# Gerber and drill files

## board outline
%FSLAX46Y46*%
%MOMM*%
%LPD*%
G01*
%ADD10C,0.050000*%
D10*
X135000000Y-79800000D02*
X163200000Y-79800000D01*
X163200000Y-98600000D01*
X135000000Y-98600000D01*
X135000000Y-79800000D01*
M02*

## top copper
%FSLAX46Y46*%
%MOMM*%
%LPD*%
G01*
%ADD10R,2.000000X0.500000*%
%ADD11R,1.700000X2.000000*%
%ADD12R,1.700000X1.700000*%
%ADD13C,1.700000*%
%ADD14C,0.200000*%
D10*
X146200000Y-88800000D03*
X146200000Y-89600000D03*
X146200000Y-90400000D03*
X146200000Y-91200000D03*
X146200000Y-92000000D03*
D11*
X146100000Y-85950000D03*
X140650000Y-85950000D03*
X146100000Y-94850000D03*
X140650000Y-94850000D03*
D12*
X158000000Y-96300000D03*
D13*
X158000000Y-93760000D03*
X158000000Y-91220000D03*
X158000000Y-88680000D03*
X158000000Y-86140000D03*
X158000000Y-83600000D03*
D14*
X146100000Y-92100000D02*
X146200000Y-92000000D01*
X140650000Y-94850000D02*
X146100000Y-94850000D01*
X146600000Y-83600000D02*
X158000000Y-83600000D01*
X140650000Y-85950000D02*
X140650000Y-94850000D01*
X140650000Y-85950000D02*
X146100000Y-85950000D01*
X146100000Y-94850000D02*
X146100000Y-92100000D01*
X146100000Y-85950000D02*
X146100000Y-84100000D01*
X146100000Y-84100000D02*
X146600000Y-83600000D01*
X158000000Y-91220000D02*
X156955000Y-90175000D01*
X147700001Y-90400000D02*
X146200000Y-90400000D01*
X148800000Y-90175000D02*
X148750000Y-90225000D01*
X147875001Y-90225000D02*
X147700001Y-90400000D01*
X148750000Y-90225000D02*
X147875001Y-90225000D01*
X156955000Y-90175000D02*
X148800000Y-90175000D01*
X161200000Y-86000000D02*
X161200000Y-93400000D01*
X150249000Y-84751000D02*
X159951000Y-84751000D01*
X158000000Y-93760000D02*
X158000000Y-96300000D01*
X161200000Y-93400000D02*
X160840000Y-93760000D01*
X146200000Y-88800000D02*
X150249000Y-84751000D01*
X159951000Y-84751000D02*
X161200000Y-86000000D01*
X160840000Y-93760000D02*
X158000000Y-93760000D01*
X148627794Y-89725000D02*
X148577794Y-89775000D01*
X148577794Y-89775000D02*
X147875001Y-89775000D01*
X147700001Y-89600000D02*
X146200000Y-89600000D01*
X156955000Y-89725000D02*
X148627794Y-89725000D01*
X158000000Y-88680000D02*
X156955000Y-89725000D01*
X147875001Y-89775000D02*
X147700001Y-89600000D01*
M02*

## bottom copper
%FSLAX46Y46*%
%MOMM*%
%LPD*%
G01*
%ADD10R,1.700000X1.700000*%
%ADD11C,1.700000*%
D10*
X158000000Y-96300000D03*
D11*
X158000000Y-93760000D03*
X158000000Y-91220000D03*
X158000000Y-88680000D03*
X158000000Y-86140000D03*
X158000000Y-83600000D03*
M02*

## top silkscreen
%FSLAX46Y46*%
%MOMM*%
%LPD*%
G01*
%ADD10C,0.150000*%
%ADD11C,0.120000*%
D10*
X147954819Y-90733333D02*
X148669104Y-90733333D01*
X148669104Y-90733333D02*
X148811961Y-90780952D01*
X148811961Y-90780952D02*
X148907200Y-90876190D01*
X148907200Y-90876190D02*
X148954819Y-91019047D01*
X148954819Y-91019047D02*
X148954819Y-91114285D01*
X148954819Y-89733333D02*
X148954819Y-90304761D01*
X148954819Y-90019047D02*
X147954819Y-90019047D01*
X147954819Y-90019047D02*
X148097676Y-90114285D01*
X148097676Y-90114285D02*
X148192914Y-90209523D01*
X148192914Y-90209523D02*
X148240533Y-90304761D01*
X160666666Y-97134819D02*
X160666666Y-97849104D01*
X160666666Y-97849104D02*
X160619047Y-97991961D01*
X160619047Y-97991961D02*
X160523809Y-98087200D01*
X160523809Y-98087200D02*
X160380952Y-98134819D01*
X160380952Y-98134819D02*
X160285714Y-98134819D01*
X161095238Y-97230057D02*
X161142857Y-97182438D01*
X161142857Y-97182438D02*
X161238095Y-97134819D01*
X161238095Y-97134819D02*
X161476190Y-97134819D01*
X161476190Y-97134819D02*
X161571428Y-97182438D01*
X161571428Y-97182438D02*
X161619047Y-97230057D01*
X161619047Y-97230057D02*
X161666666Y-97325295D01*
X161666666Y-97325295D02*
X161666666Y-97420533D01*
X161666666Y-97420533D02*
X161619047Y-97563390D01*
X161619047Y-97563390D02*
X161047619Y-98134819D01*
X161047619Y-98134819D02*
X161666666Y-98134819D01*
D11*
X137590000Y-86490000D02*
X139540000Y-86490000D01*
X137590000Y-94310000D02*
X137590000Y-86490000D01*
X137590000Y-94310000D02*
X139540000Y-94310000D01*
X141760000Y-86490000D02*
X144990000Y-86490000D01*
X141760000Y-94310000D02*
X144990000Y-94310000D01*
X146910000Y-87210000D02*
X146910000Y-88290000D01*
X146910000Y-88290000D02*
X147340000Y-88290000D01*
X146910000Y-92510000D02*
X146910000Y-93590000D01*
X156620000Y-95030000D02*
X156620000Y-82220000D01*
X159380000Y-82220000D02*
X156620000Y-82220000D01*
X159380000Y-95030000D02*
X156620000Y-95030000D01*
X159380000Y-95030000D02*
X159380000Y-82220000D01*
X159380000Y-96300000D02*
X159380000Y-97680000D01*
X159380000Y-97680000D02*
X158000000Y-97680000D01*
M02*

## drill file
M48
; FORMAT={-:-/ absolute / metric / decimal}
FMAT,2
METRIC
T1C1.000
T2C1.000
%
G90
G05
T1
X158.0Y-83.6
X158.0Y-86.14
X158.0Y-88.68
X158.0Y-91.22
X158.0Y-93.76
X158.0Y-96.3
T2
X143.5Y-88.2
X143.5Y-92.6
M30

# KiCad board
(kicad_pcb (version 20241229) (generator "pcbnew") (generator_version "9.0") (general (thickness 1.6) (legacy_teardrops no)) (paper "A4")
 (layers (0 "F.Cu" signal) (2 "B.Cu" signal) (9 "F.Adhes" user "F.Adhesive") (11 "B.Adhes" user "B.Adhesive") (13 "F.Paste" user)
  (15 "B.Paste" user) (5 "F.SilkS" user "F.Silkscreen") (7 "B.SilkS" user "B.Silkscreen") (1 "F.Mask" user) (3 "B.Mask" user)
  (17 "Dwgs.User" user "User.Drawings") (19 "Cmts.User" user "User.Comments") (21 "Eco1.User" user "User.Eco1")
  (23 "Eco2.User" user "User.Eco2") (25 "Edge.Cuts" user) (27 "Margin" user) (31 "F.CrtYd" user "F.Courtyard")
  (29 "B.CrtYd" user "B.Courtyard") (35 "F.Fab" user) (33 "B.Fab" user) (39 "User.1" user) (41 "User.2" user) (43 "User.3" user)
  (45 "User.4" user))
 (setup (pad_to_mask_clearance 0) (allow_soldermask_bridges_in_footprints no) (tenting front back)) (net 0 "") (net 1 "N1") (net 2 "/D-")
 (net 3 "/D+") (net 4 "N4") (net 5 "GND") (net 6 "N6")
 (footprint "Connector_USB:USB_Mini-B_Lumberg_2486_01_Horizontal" (layer "F.Cu") (at 143.5 90.4 -90)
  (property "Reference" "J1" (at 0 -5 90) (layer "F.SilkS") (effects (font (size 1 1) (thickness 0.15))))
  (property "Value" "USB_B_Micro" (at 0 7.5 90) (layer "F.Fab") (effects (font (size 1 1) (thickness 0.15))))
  (fp_line (start -3.91 5.91) (end -3.91 3.96) (stroke (width 0.12) (type solid)) (layer "F.SilkS"))
  (fp_line (start 3.91 5.91) (end -3.91 5.91) (stroke (width 0.12) (type solid)) (layer "F.SilkS"))
  (fp_line (start 3.91 5.91) (end 3.91 3.96) (stroke (width 0.12) (type solid)) (layer "F.SilkS"))
  (fp_line (start -3.91 1.74) (end -3.91 -1.49) (stroke (width 0.12) (type solid)) (layer "F.SilkS"))
  (fp_line (start 3.91 1.74) (end 3.91 -1.49) (stroke (width 0.12) (type solid)) (layer "F.SilkS"))
  (fp_line (start -3.19 -3.41) (end -2.11 -3.41) (stroke (width 0.12) (type solid)) (layer "F.SilkS"))
  (fp_line (start -2.11 -3.41) (end -2.11 -3.84) (stroke (width 0.12) (type solid)) (layer "F.SilkS"))
  (fp_line (start 2.11 -3.41) (end 3.19 -3.41) (stroke (width 0.12) (type solid)) (layer "F.SilkS"))
  (pad "" np_thru_hole circle (at -2.2 0 270) (size 1 1) (drill 1) (layers "*.Cu" "*.Mask"))
  (pad "" np_thru_hole circle (at 2.2 0 270) (size 1 1) (drill 1) (layers "*.Cu" "*.Mask"))
  (pad "1" smd rect (at -1.6 -2.7 270) (size 0.5 2) (layers "F.Cu" "F.Mask" "F.Paste") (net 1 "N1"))
  (pad "2" smd rect (at -0.8 -2.7 270) (size 0.5 2) (layers "F.Cu" "F.Mask" "F.Paste") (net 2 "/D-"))
  (pad "3" smd rect (at 0 -2.7 270) (size 0.5 2) (layers "F.Cu" "F.Mask" "F.Paste") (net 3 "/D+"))
  (pad "4" smd rect (at 0.8 -2.7 270) (size 0.5 2) (layers "F.Cu" "F.Mask" "F.Paste") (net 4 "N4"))
  (pad "5" smd rect (at 1.6 -2.7 270) (size 0.5 2) (layers "F.Cu" "F.Mask" "F.Paste") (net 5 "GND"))
  (pad "6" smd rect (at -4.45 -2.6 270) (size 2 1.7) (layers "F.Cu" "F.Mask" "F.Paste") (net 5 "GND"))
  (pad "6" smd rect (at -4.45 2.85 270) (size 2 1.7) (layers "F.Cu" "F.Mask" "F.Paste") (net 5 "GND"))
  (pad "6" smd rect (at 4.45 -2.6 270) (size 2 1.7) (layers "F.Cu" "F.Mask" "F.Paste") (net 5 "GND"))
  (pad "6" smd rect (at 4.45 2.85 270) (size 2 1.7) (layers "F.Cu" "F.Mask" "F.Paste") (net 5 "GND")))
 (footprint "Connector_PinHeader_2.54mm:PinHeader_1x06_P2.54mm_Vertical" (layer "F.Cu") (at 158 96.3 180)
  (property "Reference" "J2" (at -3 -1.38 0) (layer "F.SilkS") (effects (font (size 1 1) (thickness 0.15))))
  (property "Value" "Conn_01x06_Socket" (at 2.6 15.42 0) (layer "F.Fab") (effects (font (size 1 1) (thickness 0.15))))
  (fp_line (start 1.38 1.27) (end 1.38 14.08) (stroke (width 0.12) (type solid)) (layer "F.SilkS"))
  (fp_line (start -1.38 14.08) (end 1.38 14.08) (stroke (width 0.12) (type solid)) (layer "F.SilkS"))
  (fp_line (start -1.38 1.27) (end 1.38 1.27) (stroke (width 0.12) (type solid)) (layer "F.SilkS"))
  (fp_line (start -1.38 1.27) (end -1.38 14.08) (stroke (width 0.12) (type solid)) (layer "F.SilkS"))
  (fp_line (start -1.38 0) (end -1.38 -1.38) (stroke (width 0.12) (type solid)) (layer "F.SilkS"))
  (fp_line (start -1.38 -1.38) (end 0 -1.38) (stroke (width 0.12) (type solid)) (layer "F.SilkS"))
  (pad "1" thru_hole rect (at 0 0 180) (size 1.7 1.7) (drill 1) (layers "*.Cu" "*.Mask") (remove_unused_layers no) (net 1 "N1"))
  (pad "2" thru_hole circle (at 0 2.54 180) (size 1.7 1.7) (drill 1) (layers "*.Cu" "*.Mask") (remove_unused_layers no) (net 1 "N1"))
  (pad "3" thru_hole circle (at 0 5.08 180) (size 1.7 1.7) (drill 1) (layers "*.Cu" "*.Mask") (remove_unused_layers no) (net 3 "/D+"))
  (pad "4" thru_hole circle (at 0 7.62 180) (size 1.7 1.7) (drill 1) (layers "*.Cu" "*.Mask") (remove_unused_layers no) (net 2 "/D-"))
  (pad "5" thru_hole circle (at 0 10.16 180) (size 1.7 1.7) (drill 1) (layers "*.Cu" "*.Mask") (remove_unused_layers no) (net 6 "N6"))
  (pad "6" thru_hole circle (at 0 12.7 180) (size 1.7 1.7) (drill 1) (layers "*.Cu" "*.Mask") (remove_unused_layers no) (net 5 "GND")))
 (gr_rect (start 135 79.8) (end 163.2 98.6) (stroke (width 0.05) (type default)) (fill no) (layer "Edge.Cuts"))
 (segment (start 146.1 92.1) (end 146.2 92) (width 0.2) (layer "F.Cu") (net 5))
 (segment (start 140.65 94.85) (end 146.1 94.85) (width 0.2) (layer "F.Cu") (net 5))
 (segment (start 146.6 83.6) (end 158 83.6) (width 0.2) (layer "F.Cu") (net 5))
 (segment (start 140.65 85.95) (end 140.65 94.85) (width 0.2) (layer "F.Cu") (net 5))
 (segment (start 140.65 85.95) (end 146.1 85.95) (width 0.2) (layer "F.Cu") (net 5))
 (segment (start 146.1 94.85) (end 146.1 92.1) (width 0.2) (layer "F.Cu") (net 5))
 (segment (start 146.1 85.95) (end 146.1 84.1) (width 0.2) (layer "F.Cu") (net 5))
 (segment (start 146.1 84.1) (end 146.6 83.6) (width 0.2) (layer "F.Cu") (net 5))
 (segment (start 158 91.22) (end 156.955 90.175) (width 0.2) (layer "F.Cu") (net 3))
 (segment (start 147.700001 90.4) (end 146.2 90.4) (width 0.2) (layer "F.Cu") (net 3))
 (segment (start 148.8 90.175) (end 148.75 90.225) (width 0.2) (layer "F.Cu") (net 3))
 (segment (start 147.875001 90.225) (end 147.700001 90.4) (width 0.2) (layer "F.Cu") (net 3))
 (segment (start 148.75 90.225) (end 147.875001 90.225) (width 0.2) (layer "F.Cu") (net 3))
 (segment (start 156.955 90.175) (end 148.8 90.175) (width 0.2) (layer "F.Cu") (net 3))
 (segment (start 161.2 86) (end 161.2 93.4) (width 0.2) (layer "F.Cu") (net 1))
 (segment (start 150.249 84.751) (end 159.951 84.751) (width 0.2) (layer "F.Cu") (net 1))
 (segment (start 158 93.76) (end 158 96.3) (width 0.2) (layer "F.Cu") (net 1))
 (segment (start 161.2 93.4) (end 160.84 93.76) (width 0.2) (layer "F.Cu") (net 1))
 (segment (start 146.2 88.8) (end 150.249 84.751) (width 0.2) (layer "F.Cu") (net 1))
 (segment (start 159.951 84.751) (end 161.2 86) (width 0.2) (layer "F.Cu") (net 1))
 (segment (start 160.84 93.76) (end 158 93.76) (width 0.2) (layer "F.Cu") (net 1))
 (segment (start 148.627794 89.725) (end 148.577794 89.775) (width 0.2) (layer "F.Cu") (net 2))
 (segment (start 148.577794 89.775) (end 147.875001 89.775) (width 0.2) (layer "F.Cu") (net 2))
 (segment (start 147.700001 89.6) (end 146.2 89.6) (width 0.2) (layer "F.Cu") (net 2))
 (segment (start 156.955 89.725) (end 148.627794 89.725) (width 0.2) (layer "F.Cu") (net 2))
 (segment (start 158 88.68) (end 156.955 89.725) (width 0.2) (layer "F.Cu") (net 2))
 (segment (start 147.875001 89.775) (end 147.700001 89.6) (width 0.2) (layer "F.Cu") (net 2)))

